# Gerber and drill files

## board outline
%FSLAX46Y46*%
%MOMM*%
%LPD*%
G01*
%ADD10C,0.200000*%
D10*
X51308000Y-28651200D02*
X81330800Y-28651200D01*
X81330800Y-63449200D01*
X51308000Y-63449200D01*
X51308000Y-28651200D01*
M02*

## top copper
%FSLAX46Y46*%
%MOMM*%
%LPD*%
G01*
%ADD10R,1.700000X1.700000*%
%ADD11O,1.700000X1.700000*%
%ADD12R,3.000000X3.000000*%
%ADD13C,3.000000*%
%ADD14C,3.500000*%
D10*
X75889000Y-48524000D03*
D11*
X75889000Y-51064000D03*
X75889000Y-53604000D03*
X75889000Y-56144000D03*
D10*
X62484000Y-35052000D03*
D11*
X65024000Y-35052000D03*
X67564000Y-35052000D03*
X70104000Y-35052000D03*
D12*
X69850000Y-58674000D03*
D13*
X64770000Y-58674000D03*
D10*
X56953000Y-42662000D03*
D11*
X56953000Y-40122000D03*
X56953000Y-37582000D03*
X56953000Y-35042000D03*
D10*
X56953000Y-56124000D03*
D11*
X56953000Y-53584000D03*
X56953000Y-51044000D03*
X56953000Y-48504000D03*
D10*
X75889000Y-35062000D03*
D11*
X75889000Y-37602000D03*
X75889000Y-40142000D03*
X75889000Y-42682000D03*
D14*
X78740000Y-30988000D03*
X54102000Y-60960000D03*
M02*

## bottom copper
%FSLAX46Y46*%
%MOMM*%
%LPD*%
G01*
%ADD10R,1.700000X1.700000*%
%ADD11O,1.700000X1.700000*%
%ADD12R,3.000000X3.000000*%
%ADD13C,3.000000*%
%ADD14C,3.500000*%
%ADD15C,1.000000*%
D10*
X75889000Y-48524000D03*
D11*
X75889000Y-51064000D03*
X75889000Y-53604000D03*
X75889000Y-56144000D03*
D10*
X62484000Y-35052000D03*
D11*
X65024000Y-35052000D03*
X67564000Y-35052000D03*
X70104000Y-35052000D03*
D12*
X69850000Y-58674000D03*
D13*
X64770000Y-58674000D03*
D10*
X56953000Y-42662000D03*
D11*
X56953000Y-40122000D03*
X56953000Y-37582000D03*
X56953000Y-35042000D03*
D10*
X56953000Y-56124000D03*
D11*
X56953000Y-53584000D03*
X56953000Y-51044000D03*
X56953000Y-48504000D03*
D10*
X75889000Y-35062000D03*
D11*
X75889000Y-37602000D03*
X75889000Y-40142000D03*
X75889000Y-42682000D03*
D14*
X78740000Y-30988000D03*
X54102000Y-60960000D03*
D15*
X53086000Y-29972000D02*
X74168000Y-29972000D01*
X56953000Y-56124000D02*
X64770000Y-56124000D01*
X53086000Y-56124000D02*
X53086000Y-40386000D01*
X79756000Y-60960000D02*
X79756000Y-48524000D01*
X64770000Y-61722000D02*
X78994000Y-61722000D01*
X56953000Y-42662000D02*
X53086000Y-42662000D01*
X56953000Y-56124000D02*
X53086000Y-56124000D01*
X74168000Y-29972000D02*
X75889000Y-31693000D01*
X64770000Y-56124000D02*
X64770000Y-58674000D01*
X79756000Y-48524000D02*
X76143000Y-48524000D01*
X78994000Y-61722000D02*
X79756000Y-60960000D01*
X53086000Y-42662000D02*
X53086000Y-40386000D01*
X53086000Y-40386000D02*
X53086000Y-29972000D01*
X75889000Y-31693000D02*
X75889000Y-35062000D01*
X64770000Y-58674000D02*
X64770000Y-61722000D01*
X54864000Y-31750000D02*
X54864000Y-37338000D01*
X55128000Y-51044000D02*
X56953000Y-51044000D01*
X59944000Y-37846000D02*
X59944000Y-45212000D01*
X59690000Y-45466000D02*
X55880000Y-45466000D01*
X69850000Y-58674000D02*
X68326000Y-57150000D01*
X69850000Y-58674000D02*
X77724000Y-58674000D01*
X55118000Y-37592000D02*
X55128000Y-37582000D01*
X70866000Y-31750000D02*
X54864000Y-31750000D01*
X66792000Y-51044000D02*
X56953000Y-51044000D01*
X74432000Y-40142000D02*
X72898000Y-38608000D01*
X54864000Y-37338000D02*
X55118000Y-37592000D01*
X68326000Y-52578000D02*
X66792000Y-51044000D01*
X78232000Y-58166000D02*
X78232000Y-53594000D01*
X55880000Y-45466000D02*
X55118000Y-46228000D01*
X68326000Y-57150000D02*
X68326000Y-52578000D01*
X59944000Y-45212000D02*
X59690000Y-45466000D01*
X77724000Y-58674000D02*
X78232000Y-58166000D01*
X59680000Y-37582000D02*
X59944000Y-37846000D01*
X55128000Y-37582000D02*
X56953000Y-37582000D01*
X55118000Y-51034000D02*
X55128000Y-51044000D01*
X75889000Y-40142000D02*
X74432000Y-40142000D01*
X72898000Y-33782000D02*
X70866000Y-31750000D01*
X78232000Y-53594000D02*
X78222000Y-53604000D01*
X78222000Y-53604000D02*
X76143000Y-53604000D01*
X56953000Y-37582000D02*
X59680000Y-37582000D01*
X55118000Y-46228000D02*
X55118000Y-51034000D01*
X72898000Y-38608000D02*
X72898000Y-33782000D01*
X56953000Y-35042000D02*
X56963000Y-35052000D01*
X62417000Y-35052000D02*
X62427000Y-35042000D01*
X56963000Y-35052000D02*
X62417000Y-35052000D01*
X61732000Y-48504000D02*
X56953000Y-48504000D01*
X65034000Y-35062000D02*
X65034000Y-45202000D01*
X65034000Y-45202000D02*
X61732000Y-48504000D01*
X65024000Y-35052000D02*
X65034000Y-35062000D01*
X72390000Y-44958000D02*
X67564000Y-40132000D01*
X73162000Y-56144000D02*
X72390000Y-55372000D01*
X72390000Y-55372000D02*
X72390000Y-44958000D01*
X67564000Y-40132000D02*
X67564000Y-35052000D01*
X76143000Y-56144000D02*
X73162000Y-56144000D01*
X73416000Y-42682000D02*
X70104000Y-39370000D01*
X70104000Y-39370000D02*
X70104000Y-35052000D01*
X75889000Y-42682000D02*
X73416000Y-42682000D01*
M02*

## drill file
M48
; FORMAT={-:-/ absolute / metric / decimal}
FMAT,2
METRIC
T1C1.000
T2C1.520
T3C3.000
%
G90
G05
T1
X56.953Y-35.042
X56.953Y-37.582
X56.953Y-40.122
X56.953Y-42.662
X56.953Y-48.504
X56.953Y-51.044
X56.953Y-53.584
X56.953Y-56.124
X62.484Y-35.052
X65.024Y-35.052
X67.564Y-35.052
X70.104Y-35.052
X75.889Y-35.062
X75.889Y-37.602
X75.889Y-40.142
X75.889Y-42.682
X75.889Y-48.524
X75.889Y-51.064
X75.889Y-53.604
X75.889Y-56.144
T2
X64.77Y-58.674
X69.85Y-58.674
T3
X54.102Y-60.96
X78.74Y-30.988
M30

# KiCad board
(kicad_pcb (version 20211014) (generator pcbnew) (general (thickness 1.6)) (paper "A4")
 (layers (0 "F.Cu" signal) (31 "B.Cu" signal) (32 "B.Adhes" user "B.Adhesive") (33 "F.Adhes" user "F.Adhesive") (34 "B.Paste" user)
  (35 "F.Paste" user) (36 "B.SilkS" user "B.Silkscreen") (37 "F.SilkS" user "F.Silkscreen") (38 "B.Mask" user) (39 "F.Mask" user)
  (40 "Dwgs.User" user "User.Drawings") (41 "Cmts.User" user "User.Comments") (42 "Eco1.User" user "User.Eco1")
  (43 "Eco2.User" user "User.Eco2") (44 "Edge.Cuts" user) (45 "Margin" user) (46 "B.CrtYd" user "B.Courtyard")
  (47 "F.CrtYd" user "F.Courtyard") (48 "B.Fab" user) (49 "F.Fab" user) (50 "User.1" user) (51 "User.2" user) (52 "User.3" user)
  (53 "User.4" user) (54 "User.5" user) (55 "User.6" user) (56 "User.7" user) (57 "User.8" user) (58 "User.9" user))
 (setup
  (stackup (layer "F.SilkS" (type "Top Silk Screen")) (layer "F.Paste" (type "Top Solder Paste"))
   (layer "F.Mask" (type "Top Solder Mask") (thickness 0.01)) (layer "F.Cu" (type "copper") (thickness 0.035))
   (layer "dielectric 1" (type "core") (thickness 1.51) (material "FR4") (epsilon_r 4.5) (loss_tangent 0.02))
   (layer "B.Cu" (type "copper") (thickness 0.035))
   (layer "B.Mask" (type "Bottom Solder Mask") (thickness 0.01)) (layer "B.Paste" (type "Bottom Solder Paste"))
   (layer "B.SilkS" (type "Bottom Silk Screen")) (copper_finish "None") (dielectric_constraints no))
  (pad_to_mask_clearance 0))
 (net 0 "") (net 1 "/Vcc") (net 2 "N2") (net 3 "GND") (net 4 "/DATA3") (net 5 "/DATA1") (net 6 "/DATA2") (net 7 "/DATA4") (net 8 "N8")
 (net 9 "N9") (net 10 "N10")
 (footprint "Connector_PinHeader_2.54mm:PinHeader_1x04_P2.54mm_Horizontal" (layer "F.Cu") (at 75.889 48.524)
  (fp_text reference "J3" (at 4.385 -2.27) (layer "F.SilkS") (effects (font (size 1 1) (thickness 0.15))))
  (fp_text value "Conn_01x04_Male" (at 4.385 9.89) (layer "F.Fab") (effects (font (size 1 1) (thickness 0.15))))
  (pad "1" thru_hole rect (at 0 0) (size 1.7 1.7) (drill 1) (layers *.Cu *.Mask) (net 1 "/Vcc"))
  (pad "2" thru_hole oval (at 0 2.54) (size 1.7 1.7) (drill 1) (layers *.Cu *.Mask) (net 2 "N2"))
  (pad "3" thru_hole oval (at 0 5.08) (size 1.7 1.7) (drill 1) (layers *.Cu *.Mask) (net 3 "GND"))
  (pad "4" thru_hole oval (at 0 7.62) (size 1.7 1.7) (drill 1) (layers *.Cu *.Mask) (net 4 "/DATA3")))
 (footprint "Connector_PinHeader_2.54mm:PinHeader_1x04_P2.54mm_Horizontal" (layer "F.Cu") (at 62.484 35.052 90)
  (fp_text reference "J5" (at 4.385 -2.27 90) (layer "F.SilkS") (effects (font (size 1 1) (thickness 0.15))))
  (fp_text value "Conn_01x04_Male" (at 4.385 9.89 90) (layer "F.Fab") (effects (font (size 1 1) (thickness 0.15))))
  (pad "1" thru_hole rect (at 0 0 90) (size 1.7 1.7) (drill 1) (layers *.Cu *.Mask) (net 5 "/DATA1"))
  (pad "2" thru_hole oval (at 0 2.54 90) (size 1.7 1.7) (drill 1) (layers *.Cu *.Mask) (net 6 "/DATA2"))
  (pad "3" thru_hole oval (at 0 5.08 90) (size 1.7 1.7) (drill 1) (layers *.Cu *.Mask) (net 4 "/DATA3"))
  (pad "4" thru_hole oval (at 0 7.62 90) (size 1.7 1.7) (drill 1) (layers *.Cu *.Mask) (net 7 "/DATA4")))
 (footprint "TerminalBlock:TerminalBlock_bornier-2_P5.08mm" (layer "F.Cu") (at 69.85 58.674 180)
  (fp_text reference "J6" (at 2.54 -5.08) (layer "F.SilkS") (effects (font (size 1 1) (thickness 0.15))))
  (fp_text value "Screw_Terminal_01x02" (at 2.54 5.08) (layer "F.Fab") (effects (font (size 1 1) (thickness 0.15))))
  (pad "1" thru_hole rect (at 0 0 180) (size 3 3) (drill 1.52) (layers *.Cu *.Mask) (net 3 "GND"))
  (pad "2" thru_hole circle (at 5.08 0 180) (size 3 3) (drill 1.52) (layers *.Cu *.Mask) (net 1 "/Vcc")))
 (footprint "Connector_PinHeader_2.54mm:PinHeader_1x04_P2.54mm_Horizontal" (layer "F.Cu") (at 56.953 42.662 180)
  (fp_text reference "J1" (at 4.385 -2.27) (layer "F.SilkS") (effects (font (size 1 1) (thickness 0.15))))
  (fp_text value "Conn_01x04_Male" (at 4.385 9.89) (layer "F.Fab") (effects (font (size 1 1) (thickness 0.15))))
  (pad "1" thru_hole rect (at 0 0 180) (size 1.7 1.7) (drill 1) (layers *.Cu *.Mask) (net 1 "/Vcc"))
  (pad "2" thru_hole oval (at 0 2.54 180) (size 1.7 1.7) (drill 1) (layers *.Cu *.Mask) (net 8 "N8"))
  (pad "3" thru_hole oval (at 0 5.08 180) (size 1.7 1.7) (drill 1) (layers *.Cu *.Mask) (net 3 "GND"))
  (pad "4" thru_hole oval (at 0 7.62 180) (size 1.7 1.7) (drill 1) (layers *.Cu *.Mask) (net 5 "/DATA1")))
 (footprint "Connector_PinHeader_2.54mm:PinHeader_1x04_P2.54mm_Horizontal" (layer "F.Cu") (at 56.953 56.124 180)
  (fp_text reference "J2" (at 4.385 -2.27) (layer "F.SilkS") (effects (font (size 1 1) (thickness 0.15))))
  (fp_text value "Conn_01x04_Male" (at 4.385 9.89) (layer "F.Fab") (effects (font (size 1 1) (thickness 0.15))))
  (pad "1" thru_hole rect (at 0 0 180) (size 1.7 1.7) (drill 1) (layers *.Cu *.Mask) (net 1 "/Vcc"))
  (pad "2" thru_hole oval (at 0 2.54 180) (size 1.7 1.7) (drill 1) (layers *.Cu *.Mask) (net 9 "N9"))
  (pad "3" thru_hole oval (at 0 5.08 180) (size 1.7 1.7) (drill 1) (layers *.Cu *.Mask) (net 3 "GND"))
  (pad "4" thru_hole oval (at 0 7.62 180) (size 1.7 1.7) (drill 1) (layers *.Cu *.Mask) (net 6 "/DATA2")))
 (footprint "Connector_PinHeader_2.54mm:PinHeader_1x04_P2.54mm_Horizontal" (layer "F.Cu") (at 75.889 35.062)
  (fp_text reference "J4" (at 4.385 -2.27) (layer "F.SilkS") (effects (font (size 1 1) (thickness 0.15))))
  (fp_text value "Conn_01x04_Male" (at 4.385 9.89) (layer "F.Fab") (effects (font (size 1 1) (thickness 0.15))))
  (pad "1" thru_hole rect (at 0 0) (size 1.7 1.7) (drill 1) (layers *.Cu *.Mask) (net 1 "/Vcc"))
  (pad "2" thru_hole oval (at 0 2.54) (size 1.7 1.7) (drill 1) (layers *.Cu *.Mask) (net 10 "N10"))
  (pad "3" thru_hole oval (at 0 5.08) (size 1.7 1.7) (drill 1) (layers *.Cu *.Mask) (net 3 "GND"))
  (pad "4" thru_hole oval (at 0 7.62) (size 1.7 1.7) (drill 1) (layers *.Cu *.Mask) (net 7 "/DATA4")))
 (gr_rect (start 51.308 28.6512) (end 81.3308 63.4492) (layer "Edge.Cuts") (width 0.2) (fill none))
 (via (at 78.74 30.988) (size 3.5) (drill 3) (layers "F.Cu" "B.Cu") (free) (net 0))
 (via (at 54.102 60.96) (size 3.5) (drill 3) (layers "F.Cu" "B.Cu") (free) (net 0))
 (segment (start 53.086 29.972) (end 74.168 29.972) (width 1) (layer "B.Cu") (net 1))
 (segment (start 56.953 56.124) (end 64.77 56.124) (width 1) (layer "B.Cu") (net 1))
 (segment (start 53.086 56.124) (end 53.086 40.386) (width 1) (layer "B.Cu") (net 1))
 (segment (start 79.756 60.96) (end 79.756 48.524) (width 1) (layer "B.Cu") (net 1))
 (segment (start 64.77 61.722) (end 78.994 61.722) (width 1) (layer "B.Cu") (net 1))
 (segment (start 56.953 42.662) (end 53.086 42.662) (width 1) (layer "B.Cu") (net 1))
 (segment (start 56.953 56.124) (end 53.086 56.124) (width 1) (layer "B.Cu") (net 1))
 (segment (start 74.168 29.972) (end 75.889 31.693) (width 1) (layer "B.Cu") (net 1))
 (segment (start 64.77 56.124) (end 64.77 58.674) (width 1) (layer "B.Cu") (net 1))
 (segment (start 79.756 48.524) (end 76.143 48.524) (width 1) (layer "B.Cu") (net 1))
 (segment (start 78.994 61.722) (end 79.756 60.96) (width 1) (layer "B.Cu") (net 1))
 (segment (start 53.086 42.662) (end 53.086 40.386) (width 1) (layer "B.Cu") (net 1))
 (segment (start 53.086 40.386) (end 53.086 29.972) (width 1) (layer "B.Cu") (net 1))
 (segment (start 75.889 31.693) (end 75.889 35.062) (width 1) (layer "B.Cu") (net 1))
 (segment (start 64.77 58.674) (end 64.77 61.722) (width 1) (layer "B.Cu") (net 1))
 (segment (start 54.864 31.75) (end 54.864 37.338) (width 1) (layer "B.Cu") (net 3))
 (segment (start 55.128 51.044) (end 56.953 51.044) (width 1) (layer "B.Cu") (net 3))
 (segment (start 59.944 37.846) (end 59.944 45.212) (width 1) (layer "B.Cu") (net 3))
 (segment (start 59.69 45.466) (end 55.88 45.466) (width 1) (layer "B.Cu") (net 3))
 (segment (start 69.85 58.674) (end 68.326 57.15) (width 1) (layer "B.Cu") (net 3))
 (segment (start 69.85 58.674) (end 77.724 58.674) (width 1) (layer "B.Cu") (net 3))
 (segment (start 55.118 37.592) (end 55.128 37.582) (width 1) (layer "B.Cu") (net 3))
 (segment (start 70.866 31.75) (end 54.864 31.75) (width 1) (layer "B.Cu") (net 3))
 (segment (start 66.792 51.044) (end 56.953 51.044) (width 1) (layer "B.Cu") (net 3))
 (segment (start 74.432 40.142) (end 72.898 38.608) (width 1) (layer "B.Cu") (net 3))
 (segment (start 54.864 37.338) (end 55.118 37.592) (width 1) (layer "B.Cu") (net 3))
 (segment (start 68.326 52.578) (end 66.792 51.044) (width 1) (layer "B.Cu") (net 3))
 (segment (start 78.232 58.166) (end 78.232 53.594) (width 1) (layer "B.Cu") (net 3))
 (segment (start 55.88 45.466) (end 55.118 46.228) (width 1) (layer "B.Cu") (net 3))
 (segment (start 68.326 57.15) (end 68.326 52.578) (width 1) (layer "B.Cu") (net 3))
 (segment (start 59.944 45.212) (end 59.69 45.466) (width 1) (layer "B.Cu") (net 3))
 (segment (start 77.724 58.674) (end 78.232 58.166) (width 1) (layer "B.Cu") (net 3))
 (segment (start 59.68 37.582) (end 59.944 37.846) (width 1) (layer "B.Cu") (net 3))
 (segment (start 55.128 37.582) (end 56.953 37.582) (width 1) (layer "B.Cu") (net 3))
 (segment (start 55.118 51.034) (end 55.128 51.044) (width 1) (layer "B.Cu") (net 3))
 (segment (start 75.889 40.142) (end 74.432 40.142) (width 1) (layer "B.Cu") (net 3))
 (segment (start 72.898 33.782) (end 70.866 31.75) (width 1) (layer "B.Cu") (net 3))
 (segment (start 78.232 53.594) (end 78.222 53.604) (width 1) (layer "B.Cu") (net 3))
 (segment (start 78.222 53.604) (end 76.143 53.604) (width 1) (layer "B.Cu") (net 3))
 (segment (start 56.953 37.582) (end 59.68 37.582) (width 1) (layer "B.Cu") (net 3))
 (segment (start 55.118 46.228) (end 55.118 51.034) (width 1) (layer "B.Cu") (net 3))
 (segment (start 72.898 38.608) (end 72.898 33.782) (width 1) (layer "B.Cu") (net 3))
 (segment (start 56.953 35.042) (end 56.963 35.052) (width 1) (layer "B.Cu") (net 5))
 (segment (start 62.417 35.052) (end 62.427 35.042) (width 1) (layer "B.Cu") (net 5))
 (segment (start 56.963 35.052) (end 62.417 35.052) (width 1) (layer "B.Cu") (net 5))
 (segment (start 61.732 48.504) (end 56.953 48.504) (width 1) (layer "B.Cu") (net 6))
 (segment (start 65.034 35.062) (end 65.034 45.202) (width 1) (layer "B.Cu") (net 6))
 (segment (start 65.034 45.202) (end 61.732 48.504) (width 1) (layer "B.Cu") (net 6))
 (segment (start 65.024 35.052) (end 65.034 35.062) (width 1) (layer "B.Cu") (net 6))
 (segment (start 72.39 44.958) (end 67.564 40.132) (width 1) (layer "B.Cu") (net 4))
 (segment (start 73.162 56.144) (end 72.39 55.372) (width 1) (layer "B.Cu") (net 4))
 (segment (start 72.39 55.372) (end 72.39 44.958) (width 1) (layer "B.Cu") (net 4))
 (segment (start 67.564 40.132) (end 67.564 35.052) (width 1) (layer "B.Cu") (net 4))
 (segment (start 76.143 56.144) (end 73.162 56.144) (width 1) (layer "B.Cu") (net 4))
 (segment (start 73.416 42.682) (end 70.104 39.37) (width 1) (layer "B.Cu") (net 7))
 (segment (start 70.104 39.37) (end 70.104 35.052) (width 1) (layer "B.Cu") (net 7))
 (segment (start 75.889 42.682) (end 73.416 42.682) (width 1) (layer "B.Cu") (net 7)))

